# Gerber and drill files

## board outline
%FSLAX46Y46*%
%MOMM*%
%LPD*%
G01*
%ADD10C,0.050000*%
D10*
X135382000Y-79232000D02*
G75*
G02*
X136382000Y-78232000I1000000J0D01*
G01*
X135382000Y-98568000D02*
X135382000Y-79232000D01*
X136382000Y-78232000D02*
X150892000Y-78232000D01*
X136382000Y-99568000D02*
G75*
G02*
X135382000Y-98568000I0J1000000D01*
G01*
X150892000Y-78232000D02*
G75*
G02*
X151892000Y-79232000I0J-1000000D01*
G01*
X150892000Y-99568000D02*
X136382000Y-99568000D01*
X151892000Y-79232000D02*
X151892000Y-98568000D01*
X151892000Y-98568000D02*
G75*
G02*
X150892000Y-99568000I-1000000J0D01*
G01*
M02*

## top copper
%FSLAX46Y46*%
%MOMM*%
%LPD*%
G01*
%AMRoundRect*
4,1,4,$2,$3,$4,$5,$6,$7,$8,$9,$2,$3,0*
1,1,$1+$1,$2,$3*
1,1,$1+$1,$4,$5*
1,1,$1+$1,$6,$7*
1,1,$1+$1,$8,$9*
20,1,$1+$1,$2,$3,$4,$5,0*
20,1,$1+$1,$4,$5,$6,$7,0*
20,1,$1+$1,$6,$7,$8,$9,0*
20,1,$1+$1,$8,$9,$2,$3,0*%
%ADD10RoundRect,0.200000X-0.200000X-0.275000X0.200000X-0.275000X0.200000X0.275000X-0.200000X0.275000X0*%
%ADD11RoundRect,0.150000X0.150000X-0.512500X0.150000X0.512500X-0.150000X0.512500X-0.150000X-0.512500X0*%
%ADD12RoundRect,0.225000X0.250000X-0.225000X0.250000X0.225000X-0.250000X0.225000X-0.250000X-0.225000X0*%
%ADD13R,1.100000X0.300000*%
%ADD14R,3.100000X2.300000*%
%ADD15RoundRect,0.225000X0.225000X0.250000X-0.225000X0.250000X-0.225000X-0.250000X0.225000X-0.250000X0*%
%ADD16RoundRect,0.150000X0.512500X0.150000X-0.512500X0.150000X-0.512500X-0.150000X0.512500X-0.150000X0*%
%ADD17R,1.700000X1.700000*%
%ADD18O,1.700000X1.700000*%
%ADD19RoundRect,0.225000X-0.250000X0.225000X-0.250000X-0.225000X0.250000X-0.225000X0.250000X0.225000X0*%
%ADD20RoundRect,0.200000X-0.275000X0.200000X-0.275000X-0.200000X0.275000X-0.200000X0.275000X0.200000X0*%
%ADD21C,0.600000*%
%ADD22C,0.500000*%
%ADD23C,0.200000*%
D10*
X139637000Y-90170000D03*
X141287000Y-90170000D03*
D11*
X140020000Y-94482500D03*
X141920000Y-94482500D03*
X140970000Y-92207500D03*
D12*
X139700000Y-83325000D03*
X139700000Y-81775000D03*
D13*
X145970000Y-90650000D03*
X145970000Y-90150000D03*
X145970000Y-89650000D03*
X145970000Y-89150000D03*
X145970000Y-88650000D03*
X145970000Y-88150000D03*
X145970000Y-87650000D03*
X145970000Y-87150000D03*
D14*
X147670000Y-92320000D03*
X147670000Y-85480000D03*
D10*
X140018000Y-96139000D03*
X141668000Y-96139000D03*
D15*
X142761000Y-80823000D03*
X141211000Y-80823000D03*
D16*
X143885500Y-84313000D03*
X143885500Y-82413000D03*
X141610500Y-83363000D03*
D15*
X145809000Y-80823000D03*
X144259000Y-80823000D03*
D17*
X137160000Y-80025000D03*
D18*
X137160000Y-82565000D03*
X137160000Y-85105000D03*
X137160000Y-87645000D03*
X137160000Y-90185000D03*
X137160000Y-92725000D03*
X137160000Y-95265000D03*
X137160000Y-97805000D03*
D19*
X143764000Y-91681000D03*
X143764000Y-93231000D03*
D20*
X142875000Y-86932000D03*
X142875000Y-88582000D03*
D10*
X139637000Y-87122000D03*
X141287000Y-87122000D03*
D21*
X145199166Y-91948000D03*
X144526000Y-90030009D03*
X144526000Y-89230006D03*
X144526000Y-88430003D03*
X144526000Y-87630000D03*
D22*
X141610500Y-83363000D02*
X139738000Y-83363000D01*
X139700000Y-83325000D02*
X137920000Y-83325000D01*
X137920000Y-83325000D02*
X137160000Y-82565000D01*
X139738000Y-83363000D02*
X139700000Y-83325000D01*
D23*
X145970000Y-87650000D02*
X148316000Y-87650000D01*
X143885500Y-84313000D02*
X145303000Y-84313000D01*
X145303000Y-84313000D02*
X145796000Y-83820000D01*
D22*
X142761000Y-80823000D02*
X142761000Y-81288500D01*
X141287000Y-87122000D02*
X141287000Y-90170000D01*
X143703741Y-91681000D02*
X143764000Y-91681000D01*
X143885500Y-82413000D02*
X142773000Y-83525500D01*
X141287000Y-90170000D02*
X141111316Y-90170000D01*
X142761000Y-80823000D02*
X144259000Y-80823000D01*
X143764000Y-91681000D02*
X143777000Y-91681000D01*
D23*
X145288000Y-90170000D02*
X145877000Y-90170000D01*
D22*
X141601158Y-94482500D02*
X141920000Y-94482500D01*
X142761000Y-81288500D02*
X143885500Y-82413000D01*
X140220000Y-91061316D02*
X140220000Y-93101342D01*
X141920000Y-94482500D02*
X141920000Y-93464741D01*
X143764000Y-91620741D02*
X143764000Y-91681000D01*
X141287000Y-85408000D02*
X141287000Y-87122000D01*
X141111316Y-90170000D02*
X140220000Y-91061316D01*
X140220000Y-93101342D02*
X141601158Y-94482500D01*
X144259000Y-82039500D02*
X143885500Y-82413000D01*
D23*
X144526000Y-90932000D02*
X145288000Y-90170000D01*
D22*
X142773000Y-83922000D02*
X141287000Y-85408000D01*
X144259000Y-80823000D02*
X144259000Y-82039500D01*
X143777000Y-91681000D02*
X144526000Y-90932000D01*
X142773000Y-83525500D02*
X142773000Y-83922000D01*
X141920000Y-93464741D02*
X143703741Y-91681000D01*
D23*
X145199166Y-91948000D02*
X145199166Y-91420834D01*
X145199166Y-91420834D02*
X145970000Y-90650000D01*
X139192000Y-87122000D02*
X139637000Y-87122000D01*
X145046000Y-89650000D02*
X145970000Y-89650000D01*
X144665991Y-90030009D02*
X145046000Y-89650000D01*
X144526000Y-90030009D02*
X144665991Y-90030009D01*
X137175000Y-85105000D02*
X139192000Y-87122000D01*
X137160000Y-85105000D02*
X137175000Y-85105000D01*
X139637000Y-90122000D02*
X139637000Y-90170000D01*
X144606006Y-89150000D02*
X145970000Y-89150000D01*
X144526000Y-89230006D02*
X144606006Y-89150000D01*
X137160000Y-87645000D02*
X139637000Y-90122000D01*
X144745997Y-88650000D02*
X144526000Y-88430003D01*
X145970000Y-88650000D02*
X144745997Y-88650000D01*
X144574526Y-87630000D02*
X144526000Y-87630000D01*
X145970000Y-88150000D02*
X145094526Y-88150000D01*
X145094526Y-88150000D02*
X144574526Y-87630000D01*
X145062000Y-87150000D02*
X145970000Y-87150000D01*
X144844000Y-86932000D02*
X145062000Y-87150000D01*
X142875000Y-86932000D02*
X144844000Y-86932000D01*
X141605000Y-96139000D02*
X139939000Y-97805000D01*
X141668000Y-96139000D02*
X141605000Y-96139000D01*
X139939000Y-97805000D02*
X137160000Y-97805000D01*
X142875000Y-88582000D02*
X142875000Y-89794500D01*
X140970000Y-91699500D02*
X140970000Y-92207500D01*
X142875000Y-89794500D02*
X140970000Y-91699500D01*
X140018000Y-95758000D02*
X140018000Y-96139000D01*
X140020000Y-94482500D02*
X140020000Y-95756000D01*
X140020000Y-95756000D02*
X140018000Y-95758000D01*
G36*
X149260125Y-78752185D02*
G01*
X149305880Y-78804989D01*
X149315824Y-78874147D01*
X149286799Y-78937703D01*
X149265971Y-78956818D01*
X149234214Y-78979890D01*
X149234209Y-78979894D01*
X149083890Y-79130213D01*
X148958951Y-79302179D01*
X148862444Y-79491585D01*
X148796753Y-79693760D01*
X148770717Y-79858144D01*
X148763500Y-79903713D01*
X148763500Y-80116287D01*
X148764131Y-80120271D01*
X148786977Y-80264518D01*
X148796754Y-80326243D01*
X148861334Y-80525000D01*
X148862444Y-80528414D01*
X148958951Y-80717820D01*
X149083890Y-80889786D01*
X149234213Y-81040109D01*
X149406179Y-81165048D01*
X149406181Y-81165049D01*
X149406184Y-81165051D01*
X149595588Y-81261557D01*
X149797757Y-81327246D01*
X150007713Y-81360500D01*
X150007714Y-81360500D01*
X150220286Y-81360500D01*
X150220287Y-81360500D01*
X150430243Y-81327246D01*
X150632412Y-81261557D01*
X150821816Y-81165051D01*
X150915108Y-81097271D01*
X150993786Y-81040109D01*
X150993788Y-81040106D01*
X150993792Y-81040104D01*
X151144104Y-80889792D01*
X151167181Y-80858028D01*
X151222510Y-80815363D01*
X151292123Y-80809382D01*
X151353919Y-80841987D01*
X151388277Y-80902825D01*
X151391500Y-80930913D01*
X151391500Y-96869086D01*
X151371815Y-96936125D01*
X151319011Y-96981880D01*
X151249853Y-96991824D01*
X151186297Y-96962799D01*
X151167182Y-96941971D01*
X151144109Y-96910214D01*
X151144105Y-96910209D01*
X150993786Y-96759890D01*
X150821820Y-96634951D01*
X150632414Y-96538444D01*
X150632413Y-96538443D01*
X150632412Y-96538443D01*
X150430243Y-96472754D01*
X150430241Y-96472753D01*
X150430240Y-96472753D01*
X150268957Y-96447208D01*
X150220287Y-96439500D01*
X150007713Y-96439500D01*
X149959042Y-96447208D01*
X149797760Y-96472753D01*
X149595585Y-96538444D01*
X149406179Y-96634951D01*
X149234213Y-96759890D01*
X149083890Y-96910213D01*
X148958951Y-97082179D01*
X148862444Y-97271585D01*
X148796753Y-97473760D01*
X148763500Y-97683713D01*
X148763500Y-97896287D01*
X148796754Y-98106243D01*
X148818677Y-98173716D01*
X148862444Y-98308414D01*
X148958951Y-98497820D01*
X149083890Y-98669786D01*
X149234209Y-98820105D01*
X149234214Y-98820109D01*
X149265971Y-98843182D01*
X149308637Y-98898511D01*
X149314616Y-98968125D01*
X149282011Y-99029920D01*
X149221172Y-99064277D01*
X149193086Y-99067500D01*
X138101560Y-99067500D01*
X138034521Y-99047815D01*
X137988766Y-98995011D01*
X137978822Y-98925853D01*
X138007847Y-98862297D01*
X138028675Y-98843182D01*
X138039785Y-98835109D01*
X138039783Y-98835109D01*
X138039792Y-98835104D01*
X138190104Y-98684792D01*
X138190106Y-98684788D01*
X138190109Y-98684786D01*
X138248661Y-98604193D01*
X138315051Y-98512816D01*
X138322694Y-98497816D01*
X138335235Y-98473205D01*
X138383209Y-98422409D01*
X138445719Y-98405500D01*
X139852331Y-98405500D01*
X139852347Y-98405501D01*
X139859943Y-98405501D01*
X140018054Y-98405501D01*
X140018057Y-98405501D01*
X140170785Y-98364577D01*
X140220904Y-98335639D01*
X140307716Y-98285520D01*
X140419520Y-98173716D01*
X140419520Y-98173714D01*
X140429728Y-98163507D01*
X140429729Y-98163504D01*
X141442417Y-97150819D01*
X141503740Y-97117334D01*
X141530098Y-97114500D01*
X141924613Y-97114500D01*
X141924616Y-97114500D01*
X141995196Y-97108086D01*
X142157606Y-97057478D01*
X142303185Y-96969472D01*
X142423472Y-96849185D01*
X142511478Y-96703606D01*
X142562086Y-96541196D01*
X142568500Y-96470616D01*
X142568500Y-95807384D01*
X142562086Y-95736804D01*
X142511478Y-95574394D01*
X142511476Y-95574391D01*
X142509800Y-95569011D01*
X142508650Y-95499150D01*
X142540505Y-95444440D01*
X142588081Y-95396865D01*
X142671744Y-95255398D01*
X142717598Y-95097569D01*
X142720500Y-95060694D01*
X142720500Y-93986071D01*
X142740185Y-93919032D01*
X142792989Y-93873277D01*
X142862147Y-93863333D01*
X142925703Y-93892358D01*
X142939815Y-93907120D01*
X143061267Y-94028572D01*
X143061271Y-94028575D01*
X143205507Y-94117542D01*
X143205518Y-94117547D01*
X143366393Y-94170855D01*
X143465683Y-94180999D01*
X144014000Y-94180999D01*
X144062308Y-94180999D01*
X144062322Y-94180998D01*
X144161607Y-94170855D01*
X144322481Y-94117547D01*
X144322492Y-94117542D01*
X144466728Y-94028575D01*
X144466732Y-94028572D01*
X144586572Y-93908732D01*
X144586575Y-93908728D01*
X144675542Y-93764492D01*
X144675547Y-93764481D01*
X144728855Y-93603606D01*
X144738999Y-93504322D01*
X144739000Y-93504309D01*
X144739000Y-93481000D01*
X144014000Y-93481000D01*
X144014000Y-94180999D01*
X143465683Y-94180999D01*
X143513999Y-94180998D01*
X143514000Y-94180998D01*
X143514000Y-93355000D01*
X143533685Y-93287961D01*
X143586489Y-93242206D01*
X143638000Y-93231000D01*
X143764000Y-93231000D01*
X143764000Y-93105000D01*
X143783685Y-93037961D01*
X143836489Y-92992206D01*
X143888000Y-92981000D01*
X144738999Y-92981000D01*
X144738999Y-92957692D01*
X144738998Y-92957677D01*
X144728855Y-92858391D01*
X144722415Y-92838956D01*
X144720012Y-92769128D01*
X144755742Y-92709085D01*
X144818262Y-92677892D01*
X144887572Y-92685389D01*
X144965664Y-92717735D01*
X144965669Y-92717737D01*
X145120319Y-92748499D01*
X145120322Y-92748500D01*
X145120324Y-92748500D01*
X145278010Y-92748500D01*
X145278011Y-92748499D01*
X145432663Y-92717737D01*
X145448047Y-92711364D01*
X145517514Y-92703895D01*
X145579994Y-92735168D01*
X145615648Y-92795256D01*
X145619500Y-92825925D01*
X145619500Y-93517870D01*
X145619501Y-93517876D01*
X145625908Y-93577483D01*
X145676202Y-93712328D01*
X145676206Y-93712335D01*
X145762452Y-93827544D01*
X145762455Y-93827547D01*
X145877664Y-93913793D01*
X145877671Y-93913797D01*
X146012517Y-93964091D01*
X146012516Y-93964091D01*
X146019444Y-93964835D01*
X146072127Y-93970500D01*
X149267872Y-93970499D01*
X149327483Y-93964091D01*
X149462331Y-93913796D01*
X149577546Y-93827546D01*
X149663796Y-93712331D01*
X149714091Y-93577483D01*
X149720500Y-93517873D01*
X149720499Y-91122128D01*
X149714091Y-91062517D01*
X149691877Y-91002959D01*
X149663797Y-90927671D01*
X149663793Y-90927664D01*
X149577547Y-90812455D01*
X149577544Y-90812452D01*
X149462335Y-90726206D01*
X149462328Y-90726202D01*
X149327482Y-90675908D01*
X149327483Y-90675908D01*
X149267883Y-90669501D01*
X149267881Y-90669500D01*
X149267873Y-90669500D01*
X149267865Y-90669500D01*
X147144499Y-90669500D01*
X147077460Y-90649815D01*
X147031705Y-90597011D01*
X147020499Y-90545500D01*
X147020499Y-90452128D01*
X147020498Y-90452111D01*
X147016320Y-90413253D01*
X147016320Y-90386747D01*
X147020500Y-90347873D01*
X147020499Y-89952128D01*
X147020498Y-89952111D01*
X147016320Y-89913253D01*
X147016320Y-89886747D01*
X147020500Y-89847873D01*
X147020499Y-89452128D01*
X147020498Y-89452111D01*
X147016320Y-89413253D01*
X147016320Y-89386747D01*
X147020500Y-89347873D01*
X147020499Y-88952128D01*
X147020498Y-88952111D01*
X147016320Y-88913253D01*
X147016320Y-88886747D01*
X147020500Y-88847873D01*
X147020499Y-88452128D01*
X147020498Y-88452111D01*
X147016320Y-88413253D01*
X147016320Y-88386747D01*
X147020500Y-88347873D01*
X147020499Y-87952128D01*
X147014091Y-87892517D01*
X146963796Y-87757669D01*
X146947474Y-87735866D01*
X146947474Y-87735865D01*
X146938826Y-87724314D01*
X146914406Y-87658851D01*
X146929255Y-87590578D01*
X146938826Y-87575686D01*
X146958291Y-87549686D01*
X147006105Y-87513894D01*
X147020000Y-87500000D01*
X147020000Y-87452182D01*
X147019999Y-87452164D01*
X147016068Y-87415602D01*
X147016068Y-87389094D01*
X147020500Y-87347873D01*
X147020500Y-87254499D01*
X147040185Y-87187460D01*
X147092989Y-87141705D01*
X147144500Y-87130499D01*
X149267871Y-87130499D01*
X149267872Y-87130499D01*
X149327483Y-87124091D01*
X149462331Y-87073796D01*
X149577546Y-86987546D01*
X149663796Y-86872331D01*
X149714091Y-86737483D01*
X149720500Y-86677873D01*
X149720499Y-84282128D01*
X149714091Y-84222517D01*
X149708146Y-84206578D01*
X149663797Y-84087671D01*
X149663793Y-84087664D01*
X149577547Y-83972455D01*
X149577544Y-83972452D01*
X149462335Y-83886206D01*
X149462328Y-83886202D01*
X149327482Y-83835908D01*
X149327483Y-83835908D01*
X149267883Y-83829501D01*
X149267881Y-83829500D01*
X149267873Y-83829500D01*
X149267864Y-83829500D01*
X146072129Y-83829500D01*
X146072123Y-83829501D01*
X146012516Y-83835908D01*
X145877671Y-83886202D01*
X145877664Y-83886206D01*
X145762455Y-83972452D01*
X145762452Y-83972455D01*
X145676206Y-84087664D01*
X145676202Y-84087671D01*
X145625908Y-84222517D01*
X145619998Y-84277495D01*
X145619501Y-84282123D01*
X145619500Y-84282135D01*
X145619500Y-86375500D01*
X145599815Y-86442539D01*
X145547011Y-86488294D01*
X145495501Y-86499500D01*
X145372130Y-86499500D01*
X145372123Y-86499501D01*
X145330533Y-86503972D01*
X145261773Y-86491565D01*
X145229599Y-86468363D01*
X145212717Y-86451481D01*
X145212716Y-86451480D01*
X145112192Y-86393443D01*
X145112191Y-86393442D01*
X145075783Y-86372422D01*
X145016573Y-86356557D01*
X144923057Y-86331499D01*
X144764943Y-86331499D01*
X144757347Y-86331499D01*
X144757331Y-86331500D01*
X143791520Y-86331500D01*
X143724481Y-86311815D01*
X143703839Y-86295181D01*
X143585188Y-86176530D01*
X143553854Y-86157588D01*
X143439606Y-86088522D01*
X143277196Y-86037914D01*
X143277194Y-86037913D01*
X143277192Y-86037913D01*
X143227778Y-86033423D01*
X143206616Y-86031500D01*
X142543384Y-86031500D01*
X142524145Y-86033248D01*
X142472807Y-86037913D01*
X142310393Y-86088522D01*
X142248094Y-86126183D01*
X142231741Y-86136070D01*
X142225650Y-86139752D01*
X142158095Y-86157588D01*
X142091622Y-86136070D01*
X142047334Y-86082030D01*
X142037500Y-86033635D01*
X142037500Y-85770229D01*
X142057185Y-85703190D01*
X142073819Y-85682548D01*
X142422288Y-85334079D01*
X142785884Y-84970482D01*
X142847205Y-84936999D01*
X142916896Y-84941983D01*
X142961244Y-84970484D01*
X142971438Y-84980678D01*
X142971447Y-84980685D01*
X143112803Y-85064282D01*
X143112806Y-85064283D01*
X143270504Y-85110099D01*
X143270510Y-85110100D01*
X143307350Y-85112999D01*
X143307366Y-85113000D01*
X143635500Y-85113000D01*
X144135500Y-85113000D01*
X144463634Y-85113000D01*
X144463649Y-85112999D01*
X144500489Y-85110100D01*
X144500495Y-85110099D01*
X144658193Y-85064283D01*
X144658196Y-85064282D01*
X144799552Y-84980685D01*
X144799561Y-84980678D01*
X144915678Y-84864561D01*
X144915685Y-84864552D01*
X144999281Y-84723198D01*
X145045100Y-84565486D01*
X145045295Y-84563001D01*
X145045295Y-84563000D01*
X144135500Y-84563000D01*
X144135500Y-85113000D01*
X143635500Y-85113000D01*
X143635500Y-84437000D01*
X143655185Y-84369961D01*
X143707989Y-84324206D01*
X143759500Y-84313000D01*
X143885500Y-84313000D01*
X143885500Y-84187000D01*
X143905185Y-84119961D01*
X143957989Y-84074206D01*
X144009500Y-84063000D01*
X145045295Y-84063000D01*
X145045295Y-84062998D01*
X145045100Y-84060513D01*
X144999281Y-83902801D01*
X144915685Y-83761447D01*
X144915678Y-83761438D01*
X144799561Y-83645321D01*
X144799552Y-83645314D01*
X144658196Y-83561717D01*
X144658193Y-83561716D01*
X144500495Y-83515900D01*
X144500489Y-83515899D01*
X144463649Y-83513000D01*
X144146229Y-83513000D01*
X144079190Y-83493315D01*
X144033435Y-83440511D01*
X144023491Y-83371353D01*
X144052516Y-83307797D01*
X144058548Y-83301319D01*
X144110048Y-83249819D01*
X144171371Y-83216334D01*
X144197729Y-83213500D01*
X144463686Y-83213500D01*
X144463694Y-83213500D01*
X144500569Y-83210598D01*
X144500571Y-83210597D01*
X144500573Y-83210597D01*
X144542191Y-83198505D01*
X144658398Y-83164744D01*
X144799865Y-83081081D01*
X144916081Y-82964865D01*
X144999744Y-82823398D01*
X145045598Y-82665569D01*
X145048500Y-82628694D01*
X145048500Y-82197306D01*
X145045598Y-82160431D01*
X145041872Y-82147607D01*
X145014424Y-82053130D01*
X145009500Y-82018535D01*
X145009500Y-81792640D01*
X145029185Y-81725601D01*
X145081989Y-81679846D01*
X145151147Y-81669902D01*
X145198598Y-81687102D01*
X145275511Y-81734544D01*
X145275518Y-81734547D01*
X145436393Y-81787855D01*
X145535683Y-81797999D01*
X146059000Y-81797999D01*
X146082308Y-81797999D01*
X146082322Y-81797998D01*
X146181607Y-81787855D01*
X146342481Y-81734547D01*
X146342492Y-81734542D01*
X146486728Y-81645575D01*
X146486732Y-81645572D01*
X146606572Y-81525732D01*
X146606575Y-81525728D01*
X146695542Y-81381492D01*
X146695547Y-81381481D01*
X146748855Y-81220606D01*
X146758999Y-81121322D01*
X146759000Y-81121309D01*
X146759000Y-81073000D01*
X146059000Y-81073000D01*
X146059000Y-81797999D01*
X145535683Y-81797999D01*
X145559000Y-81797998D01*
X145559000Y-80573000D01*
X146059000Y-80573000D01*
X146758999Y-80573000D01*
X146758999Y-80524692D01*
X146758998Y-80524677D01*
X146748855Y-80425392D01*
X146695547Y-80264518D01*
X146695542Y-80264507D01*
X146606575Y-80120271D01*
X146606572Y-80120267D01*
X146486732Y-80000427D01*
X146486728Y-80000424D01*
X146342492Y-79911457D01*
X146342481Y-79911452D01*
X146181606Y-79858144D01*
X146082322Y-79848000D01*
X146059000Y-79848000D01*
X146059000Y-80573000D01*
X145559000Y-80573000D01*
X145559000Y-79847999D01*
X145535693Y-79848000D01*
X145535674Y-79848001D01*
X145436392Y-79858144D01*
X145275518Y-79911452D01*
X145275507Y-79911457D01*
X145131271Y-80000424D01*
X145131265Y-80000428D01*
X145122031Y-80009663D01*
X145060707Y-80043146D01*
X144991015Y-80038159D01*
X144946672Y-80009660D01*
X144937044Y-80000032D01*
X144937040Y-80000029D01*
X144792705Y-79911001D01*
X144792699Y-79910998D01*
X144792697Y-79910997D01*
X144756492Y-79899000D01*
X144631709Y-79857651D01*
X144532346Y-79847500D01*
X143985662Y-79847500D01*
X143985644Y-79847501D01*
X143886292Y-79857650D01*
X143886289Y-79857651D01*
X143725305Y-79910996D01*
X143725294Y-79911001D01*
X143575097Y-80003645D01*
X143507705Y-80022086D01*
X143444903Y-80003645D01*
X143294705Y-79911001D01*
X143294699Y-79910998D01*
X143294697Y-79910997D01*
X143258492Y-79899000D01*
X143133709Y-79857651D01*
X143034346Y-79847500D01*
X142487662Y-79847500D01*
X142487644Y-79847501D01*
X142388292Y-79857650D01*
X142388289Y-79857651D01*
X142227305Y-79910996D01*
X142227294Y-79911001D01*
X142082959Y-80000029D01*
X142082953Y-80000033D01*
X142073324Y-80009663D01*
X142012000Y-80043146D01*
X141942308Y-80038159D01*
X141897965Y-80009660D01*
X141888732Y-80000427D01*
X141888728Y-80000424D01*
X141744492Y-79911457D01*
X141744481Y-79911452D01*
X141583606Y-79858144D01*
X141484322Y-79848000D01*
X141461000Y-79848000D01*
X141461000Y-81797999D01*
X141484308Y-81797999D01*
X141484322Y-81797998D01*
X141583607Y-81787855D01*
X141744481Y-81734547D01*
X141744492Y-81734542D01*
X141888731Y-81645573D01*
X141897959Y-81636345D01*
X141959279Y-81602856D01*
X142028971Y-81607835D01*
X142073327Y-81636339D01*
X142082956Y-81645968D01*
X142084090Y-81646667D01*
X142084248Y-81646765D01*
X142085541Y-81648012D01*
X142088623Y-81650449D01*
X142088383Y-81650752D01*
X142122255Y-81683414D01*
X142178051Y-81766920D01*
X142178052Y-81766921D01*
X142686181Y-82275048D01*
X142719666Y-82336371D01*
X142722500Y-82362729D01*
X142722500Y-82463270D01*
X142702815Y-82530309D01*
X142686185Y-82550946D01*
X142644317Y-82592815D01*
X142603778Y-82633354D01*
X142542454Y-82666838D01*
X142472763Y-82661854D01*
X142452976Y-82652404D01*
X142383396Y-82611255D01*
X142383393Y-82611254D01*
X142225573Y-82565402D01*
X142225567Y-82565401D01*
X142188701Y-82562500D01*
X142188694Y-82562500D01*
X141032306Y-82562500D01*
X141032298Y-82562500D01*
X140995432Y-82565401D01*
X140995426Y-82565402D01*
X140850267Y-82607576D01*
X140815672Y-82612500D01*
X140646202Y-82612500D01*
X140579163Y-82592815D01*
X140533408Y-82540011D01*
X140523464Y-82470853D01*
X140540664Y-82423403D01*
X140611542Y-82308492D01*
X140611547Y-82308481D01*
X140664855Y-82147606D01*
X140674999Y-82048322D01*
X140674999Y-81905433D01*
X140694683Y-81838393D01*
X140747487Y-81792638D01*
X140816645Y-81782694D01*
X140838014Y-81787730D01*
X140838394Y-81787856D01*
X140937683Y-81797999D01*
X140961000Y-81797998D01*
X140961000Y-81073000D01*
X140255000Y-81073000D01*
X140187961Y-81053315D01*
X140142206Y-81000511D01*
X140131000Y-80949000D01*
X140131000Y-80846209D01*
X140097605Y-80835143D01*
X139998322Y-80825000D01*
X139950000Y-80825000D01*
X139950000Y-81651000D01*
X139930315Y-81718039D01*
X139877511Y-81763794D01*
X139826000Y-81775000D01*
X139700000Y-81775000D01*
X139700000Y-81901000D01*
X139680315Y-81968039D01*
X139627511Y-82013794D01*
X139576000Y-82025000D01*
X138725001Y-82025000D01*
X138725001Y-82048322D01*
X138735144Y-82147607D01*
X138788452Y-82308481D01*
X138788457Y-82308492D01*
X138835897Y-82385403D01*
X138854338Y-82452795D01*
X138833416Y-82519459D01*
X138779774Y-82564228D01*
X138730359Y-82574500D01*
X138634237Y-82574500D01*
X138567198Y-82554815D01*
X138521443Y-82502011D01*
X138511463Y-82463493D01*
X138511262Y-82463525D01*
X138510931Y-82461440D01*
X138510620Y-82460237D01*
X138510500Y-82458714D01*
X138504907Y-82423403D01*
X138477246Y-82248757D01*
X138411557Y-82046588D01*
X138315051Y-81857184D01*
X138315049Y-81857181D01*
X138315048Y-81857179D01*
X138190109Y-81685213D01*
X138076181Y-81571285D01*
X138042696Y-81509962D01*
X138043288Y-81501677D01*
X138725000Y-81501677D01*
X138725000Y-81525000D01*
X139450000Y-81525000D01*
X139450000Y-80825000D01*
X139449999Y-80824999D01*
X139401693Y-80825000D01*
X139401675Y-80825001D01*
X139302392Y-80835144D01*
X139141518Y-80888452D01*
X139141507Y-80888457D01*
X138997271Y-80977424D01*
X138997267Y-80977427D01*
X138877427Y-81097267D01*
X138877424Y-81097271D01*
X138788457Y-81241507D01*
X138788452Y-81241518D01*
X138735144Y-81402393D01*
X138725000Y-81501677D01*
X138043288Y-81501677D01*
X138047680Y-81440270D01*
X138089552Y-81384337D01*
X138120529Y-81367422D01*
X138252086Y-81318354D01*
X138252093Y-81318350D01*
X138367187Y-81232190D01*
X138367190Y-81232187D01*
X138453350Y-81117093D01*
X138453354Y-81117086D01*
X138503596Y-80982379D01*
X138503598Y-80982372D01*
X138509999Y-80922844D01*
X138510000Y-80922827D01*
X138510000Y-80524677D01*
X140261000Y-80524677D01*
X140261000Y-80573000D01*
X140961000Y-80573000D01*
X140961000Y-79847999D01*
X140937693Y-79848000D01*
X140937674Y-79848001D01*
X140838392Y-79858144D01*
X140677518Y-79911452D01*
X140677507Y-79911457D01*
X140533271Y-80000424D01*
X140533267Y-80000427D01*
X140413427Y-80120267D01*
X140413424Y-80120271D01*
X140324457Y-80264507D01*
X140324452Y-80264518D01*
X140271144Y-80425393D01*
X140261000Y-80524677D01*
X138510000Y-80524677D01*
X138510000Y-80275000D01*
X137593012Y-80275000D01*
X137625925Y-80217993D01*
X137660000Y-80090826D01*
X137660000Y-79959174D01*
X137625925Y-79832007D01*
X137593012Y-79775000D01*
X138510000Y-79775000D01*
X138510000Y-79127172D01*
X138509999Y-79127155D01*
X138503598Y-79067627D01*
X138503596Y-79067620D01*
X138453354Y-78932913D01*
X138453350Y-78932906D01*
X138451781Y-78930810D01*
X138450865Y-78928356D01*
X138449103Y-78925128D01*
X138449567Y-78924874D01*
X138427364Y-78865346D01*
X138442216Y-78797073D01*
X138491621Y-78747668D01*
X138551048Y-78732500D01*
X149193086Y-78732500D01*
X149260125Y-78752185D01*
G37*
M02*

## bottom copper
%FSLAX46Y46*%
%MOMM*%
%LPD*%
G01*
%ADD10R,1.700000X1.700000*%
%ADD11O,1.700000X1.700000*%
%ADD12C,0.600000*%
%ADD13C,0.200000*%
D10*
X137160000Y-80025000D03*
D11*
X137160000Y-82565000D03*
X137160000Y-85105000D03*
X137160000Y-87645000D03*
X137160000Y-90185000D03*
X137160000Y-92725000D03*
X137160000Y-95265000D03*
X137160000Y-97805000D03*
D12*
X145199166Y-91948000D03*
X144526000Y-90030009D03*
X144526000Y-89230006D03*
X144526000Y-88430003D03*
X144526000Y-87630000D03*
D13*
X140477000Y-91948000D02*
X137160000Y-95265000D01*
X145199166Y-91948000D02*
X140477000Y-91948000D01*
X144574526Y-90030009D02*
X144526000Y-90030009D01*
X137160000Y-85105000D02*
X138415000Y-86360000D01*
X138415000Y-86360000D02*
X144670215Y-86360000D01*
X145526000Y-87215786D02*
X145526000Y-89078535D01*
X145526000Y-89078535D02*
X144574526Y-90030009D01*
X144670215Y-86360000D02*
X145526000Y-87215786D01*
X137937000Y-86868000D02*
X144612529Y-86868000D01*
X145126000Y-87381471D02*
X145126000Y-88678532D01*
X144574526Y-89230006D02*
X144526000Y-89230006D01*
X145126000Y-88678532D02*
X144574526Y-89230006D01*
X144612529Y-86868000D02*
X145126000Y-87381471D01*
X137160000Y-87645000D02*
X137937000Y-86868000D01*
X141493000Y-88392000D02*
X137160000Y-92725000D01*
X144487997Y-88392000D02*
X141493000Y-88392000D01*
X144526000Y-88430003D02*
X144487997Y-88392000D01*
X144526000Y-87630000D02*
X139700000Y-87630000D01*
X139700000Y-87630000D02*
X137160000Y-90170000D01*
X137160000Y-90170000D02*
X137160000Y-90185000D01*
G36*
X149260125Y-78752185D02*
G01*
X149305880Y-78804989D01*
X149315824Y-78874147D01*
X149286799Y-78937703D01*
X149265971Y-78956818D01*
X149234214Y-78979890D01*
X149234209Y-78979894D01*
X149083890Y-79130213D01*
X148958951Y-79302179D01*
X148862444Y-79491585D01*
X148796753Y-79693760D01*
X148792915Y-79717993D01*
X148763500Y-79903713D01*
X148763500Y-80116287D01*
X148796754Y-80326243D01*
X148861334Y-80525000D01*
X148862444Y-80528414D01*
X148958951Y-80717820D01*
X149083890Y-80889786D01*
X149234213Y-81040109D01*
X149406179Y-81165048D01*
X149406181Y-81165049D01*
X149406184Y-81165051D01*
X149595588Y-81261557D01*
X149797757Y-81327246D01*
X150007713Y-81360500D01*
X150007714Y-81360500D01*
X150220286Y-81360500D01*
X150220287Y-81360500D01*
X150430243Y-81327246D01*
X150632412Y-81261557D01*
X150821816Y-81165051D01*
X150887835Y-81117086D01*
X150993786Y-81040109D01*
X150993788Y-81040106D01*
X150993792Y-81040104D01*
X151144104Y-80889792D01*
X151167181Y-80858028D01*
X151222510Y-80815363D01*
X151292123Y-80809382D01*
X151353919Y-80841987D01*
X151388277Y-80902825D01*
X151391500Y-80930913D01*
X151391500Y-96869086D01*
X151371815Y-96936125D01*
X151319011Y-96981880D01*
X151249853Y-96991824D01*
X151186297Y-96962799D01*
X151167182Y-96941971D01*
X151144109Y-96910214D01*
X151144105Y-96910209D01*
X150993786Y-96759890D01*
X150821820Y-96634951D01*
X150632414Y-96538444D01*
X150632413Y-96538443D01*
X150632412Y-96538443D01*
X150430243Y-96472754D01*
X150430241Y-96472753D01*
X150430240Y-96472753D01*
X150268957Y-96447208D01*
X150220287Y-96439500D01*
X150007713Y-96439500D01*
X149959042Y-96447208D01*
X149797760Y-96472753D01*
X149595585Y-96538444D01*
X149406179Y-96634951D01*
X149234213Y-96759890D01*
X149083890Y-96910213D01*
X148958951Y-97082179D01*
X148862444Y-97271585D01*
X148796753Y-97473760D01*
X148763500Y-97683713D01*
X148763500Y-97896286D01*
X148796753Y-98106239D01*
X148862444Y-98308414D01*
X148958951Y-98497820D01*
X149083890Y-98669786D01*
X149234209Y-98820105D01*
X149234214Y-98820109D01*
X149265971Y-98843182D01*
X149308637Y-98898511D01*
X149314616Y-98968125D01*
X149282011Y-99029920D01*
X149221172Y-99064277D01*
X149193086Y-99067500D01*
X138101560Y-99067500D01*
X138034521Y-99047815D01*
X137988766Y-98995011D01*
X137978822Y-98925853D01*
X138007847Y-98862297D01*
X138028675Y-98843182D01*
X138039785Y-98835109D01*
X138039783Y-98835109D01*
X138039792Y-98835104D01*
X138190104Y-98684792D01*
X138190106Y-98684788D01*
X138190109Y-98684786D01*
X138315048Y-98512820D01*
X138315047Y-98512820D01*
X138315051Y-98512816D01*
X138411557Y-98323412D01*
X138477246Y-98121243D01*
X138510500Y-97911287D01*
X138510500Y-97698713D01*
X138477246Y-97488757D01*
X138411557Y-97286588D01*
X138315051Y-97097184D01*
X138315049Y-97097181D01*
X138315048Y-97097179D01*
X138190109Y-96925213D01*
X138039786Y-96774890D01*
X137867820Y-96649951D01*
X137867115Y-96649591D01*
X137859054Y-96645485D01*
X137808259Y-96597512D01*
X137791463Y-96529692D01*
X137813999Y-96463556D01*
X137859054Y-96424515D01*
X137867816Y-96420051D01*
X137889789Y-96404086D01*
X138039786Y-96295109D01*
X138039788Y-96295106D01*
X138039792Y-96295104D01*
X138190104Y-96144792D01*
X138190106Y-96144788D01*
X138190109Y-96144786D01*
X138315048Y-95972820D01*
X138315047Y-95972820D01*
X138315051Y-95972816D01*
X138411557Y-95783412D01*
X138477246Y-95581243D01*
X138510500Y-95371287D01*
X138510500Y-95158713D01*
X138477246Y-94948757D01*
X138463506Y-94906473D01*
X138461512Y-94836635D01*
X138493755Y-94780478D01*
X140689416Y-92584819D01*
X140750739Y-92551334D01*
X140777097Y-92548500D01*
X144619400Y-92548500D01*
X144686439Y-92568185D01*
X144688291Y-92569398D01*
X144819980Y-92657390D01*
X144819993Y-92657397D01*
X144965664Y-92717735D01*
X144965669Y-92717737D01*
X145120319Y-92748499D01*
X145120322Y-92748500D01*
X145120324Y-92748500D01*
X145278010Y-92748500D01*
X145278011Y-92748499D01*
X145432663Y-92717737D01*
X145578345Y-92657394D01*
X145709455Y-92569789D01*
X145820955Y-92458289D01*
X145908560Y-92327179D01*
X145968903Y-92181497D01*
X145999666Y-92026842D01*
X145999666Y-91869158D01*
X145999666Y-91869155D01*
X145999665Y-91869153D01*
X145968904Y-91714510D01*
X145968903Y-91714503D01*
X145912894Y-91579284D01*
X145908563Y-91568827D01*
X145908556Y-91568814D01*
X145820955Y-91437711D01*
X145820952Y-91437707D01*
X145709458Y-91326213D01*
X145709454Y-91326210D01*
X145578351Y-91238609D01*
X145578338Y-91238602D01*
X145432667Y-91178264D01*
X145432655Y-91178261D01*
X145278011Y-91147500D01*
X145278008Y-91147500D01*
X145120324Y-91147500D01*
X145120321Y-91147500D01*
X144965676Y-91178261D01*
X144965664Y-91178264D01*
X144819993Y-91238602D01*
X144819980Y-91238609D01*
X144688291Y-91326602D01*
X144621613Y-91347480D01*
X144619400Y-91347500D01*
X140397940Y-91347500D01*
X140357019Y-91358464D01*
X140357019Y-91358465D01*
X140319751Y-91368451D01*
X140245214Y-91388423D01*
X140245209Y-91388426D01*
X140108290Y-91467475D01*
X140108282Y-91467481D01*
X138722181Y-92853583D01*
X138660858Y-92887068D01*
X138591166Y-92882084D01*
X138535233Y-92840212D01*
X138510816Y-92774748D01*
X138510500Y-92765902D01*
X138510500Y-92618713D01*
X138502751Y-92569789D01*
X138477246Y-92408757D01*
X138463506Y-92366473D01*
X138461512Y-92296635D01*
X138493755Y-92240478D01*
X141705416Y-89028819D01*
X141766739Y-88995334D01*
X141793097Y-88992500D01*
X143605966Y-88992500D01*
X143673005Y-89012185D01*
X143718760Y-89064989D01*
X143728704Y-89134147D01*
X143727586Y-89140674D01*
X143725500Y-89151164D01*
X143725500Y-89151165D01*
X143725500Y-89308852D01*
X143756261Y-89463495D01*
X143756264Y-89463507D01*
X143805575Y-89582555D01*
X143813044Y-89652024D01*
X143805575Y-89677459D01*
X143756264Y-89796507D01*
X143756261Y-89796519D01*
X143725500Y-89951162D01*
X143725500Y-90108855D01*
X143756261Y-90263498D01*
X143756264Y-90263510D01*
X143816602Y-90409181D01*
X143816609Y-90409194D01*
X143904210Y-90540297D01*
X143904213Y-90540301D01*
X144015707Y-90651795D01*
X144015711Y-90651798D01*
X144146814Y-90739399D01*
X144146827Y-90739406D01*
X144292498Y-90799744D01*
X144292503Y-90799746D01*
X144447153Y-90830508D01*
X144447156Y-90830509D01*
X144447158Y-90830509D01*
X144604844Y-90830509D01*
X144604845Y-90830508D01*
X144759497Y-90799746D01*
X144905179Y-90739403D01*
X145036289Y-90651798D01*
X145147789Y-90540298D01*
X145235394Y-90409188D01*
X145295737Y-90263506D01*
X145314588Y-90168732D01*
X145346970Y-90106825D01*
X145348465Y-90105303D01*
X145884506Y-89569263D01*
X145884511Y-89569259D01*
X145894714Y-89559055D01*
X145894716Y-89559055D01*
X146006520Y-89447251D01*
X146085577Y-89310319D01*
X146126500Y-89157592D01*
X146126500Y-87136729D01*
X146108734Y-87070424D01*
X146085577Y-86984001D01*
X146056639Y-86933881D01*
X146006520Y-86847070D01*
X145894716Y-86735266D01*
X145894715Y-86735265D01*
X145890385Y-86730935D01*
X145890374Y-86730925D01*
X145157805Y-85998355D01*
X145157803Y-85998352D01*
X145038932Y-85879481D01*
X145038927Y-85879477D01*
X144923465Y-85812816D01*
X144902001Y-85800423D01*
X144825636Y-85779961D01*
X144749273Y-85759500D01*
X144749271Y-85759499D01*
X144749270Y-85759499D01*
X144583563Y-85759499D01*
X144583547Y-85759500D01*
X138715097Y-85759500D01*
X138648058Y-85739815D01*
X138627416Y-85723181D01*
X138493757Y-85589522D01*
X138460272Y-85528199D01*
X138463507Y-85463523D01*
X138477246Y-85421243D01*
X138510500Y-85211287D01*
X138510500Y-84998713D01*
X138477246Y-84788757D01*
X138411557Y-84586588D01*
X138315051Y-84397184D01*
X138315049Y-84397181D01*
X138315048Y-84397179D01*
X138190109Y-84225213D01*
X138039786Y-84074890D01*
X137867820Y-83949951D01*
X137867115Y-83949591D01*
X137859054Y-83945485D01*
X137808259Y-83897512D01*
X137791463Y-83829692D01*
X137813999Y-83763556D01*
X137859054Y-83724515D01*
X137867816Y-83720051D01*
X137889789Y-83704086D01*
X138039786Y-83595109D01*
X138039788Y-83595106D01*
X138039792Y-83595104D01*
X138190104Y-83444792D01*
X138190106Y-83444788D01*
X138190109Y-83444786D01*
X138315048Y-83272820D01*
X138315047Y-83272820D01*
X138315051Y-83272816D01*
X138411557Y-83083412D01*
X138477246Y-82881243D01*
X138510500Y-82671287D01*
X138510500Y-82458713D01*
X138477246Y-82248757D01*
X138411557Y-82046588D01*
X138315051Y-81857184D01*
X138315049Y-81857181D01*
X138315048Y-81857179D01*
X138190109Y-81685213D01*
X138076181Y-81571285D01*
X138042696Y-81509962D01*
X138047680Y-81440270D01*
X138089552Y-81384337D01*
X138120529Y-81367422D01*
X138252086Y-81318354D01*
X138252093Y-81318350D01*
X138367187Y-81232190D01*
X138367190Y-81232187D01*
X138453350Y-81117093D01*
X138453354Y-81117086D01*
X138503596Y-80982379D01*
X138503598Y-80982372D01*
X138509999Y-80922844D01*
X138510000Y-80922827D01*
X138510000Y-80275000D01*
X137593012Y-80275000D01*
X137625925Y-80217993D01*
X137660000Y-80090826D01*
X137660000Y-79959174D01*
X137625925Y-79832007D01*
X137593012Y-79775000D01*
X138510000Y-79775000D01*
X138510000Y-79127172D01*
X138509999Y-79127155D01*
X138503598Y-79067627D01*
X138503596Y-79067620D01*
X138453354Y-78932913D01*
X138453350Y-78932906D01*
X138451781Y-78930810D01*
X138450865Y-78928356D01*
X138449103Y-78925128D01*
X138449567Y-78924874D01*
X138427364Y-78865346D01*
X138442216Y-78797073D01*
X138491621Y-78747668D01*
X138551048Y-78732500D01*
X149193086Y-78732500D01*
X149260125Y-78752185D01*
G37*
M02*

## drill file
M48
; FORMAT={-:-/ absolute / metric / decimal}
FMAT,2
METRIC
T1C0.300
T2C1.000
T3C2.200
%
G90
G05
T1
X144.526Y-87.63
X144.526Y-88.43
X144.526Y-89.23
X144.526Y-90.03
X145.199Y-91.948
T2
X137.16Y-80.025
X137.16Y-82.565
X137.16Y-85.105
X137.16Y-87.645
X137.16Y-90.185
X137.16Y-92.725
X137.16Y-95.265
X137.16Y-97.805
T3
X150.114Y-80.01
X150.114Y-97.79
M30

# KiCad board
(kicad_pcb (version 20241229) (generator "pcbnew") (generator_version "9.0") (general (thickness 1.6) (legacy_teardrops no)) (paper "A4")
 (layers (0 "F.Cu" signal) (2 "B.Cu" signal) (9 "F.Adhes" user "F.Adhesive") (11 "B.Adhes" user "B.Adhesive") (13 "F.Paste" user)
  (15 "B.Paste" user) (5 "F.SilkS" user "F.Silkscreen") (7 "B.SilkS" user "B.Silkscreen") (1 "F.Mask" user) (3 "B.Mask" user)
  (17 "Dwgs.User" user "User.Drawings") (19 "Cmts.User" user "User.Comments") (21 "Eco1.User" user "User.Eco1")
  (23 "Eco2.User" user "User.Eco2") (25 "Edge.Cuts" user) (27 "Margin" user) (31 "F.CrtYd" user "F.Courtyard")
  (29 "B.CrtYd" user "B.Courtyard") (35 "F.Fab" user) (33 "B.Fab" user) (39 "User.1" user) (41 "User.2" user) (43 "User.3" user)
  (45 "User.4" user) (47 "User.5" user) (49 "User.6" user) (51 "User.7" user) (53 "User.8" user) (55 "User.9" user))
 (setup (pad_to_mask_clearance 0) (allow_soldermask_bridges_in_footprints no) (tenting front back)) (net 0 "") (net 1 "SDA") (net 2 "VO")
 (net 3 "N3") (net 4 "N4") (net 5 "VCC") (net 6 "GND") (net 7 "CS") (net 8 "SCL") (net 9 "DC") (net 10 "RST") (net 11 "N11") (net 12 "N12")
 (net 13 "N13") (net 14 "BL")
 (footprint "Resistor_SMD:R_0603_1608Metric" (layer "F.Cu") (at 140.462 90.17)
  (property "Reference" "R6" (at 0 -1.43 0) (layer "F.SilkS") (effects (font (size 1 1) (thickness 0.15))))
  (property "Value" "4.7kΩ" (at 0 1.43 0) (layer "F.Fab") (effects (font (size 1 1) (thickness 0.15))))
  (pad "1" smd roundrect (at -0.825 0) (size 0.8 0.95) (layers "F.Cu" "F.Mask" "F.Paste") (roundrect_rratio 0.25) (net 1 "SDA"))
  (pad "2" smd roundrect (at 0.825 0) (size 0.8 0.95) (layers "F.Cu" "F.Mask" "F.Paste") (roundrect_rratio 0.25) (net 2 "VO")))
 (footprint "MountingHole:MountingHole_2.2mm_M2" (layer "F.Cu") (at 150.114 97.79)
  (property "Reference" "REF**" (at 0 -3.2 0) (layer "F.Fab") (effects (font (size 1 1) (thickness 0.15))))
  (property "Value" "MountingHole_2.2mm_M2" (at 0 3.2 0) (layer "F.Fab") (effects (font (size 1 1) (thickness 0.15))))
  (pad "" np_thru_hole circle (at 0 0) (size 2.2 2.2) (drill 2.2) (layers "*.Cu" "*.Mask")))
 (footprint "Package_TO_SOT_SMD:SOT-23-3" (layer "F.Cu") (at 140.97 93.345 90)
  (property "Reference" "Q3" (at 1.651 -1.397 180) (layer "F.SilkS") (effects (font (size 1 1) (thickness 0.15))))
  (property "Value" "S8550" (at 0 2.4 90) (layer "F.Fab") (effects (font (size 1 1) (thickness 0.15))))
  (pad "1" smd roundrect (at -1.1375 -0.95 90) (size 1.325 0.6) (layers "F.Cu" "F.Mask" "F.Paste") (roundrect_rratio 0.25) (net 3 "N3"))
  (pad "2" smd roundrect (at -1.1375 0.95 90) (size 1.325 0.6) (layers "F.Cu" "F.Mask" "F.Paste") (roundrect_rratio 0.25) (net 2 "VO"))
  (pad "3" smd roundrect (at 1.1375 0 90) (size 1.325 0.6) (layers "F.Cu" "F.Mask" "F.Paste") (roundrect_rratio 0.25) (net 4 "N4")))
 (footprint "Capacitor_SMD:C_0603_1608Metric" (layer "F.Cu") (at 139.7 82.55 90)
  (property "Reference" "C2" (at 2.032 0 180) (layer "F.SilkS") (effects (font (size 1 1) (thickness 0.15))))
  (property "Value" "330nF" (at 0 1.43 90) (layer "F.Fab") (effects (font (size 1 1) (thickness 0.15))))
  (pad "1" smd roundrect (at -0.775 0 90) (size 0.9 0.95) (layers "F.Cu" "F.Mask" "F.Paste") (roundrect_rratio 0.25) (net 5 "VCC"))
  (pad "2" smd roundrect (at 0.775 0 90) (size 0.9 0.95) (layers "F.Cu" "F.Mask" "F.Paste") (roundrect_rratio 0.25) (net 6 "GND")))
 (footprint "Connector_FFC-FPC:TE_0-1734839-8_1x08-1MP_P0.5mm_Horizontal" (layer "F.Cu") (at 147.32 88.9 90)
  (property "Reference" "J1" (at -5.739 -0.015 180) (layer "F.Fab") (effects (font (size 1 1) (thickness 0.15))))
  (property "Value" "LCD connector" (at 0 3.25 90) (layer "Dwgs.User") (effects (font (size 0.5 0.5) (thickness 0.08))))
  (pad "1" smd rect (at -1.75 -1.35 90) (size 0.3 1.1) (layers "F.Cu" "F.Mask" "F.Paste") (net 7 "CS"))
  (pad "2" smd rect (at -1.25 -1.35 90) (size 0.3 1.1) (layers "F.Cu" "F.Mask" "F.Paste") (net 2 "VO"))
  (pad "3" smd rect (at -0.75 -1.35 90) (size 0.3 1.1) (layers "F.Cu" "F.Mask" "F.Paste") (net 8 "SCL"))
  (pad "4" smd rect (at -0.25 -1.35 90) (size 0.3 1.1) (layers "F.Cu" "F.Mask" "F.Paste") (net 1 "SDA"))
  (pad "5" smd rect (at 0.25 -1.35 90) (size 0.3 1.1) (layers "F.Cu" "F.Mask" "F.Paste") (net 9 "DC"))
  (pad "6" smd rect (at 0.75 -1.35 90) (size 0.3 1.1) (layers "F.Cu" "F.Mask" "F.Paste") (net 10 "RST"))
  (pad "7" smd rect (at 1.25 -1.35 90) (size 0.3 1.1) (layers "F.Cu" "F.Mask" "F.Paste") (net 6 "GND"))
  (pad "8" smd rect (at 1.75 -1.35 90) (size 0.3 1.1) (layers "F.Cu" "F.Mask" "F.Paste") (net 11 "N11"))
  (pad "MP" smd rect (at -3.42 0.35 90) (size 2.3 3.1) (layers "F.Cu" "F.Mask" "F.Paste") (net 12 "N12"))
  (pad "MP" smd rect (at 3.42 0.35 90) (size 2.3 3.1) (layers "F.Cu" "F.Mask" "F.Paste") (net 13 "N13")))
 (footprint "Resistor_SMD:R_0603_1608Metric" (layer "F.Cu") (at 140.843 96.139)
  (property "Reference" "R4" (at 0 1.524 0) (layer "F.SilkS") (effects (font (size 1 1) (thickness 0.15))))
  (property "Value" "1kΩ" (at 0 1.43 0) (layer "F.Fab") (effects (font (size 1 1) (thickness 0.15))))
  (pad "1" smd roundrect (at -0.825 0) (size 0.8 0.95) (layers "F.Cu" "F.Mask" "F.Paste") (roundrect_rratio 0.25) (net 3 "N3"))
  (pad "2" smd roundrect (at 0.825 0) (size 0.8 0.95) (layers "F.Cu" "F.Mask" "F.Paste") (roundrect_rratio 0.25) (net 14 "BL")))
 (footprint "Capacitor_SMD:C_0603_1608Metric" (layer "F.Cu") (at 141.986 80.823 180)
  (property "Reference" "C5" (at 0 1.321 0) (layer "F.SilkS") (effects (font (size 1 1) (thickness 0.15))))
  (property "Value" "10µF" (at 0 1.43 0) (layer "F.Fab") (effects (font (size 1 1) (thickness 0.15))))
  (pad "1" smd roundrect (at -0.775 0 180) (size 0.9 0.95) (layers "F.Cu" "F.Mask" "F.Paste") (roundrect_rratio 0.25) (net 2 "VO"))
  (pad "2" smd roundrect (at 0.775 0 180) (size 0.9 0.95) (layers "F.Cu" "F.Mask" "F.Paste") (roundrect_rratio 0.25) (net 6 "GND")))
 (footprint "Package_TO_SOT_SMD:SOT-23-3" (layer "F.Cu") (at 142.748 83.363 180)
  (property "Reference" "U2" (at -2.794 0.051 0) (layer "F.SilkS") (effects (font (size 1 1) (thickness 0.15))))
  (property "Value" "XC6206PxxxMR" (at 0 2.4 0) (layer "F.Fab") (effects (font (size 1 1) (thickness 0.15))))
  (pad "1" smd roundrect (at -1.1375 -0.95 180) (size 1.325 0.6) (layers "F.Cu" "F.Mask" "F.Paste") (roundrect_rratio 0.25) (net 6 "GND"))
  (pad "2" smd roundrect (at -1.1375 0.95 180) (size 1.325 0.6) (layers "F.Cu" "F.Mask" "F.Paste") (roundrect_rratio 0.25) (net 2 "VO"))
  (pad "3" smd roundrect (at 1.1375 0 180) (size 1.325 0.6) (layers "F.Cu" "F.Mask" "F.Paste") (roundrect_rratio 0.25) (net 5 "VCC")))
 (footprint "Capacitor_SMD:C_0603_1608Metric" (layer "F.Cu") (at 145.034 80.823 180)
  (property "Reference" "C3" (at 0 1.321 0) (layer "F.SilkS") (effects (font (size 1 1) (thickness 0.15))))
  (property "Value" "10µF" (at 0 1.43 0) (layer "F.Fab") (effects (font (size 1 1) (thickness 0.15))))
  (pad "1" smd roundrect (at -0.775 0 180) (size 0.9 0.95) (layers "F.Cu" "F.Mask" "F.Paste") (roundrect_rratio 0.25) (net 6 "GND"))
  (pad "2" smd roundrect (at 0.775 0 180) (size 0.9 0.95) (layers "F.Cu" "F.Mask" "F.Paste") (roundrect_rratio 0.25) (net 2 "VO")))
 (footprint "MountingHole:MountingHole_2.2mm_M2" (layer "F.Cu") (at 150.114 80.01)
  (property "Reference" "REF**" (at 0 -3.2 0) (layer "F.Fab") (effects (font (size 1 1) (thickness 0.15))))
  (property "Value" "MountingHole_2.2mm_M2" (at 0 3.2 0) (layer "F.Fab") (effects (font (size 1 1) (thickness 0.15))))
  (pad "" np_thru_hole circle (at 0 0) (size 2.2 2.2) (drill 2.2) (layers "*.Cu" "*.Mask")))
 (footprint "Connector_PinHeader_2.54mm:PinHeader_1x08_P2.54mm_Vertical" (layer "F.Cu") (at 137.16 80.025)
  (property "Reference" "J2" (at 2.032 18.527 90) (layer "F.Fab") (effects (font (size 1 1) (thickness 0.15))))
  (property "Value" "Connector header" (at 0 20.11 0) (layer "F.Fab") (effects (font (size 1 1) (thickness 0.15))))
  (pad "1" thru_hole rect (at 0 0) (size 1.7 1.7) (drill 1) (layers "*.Cu" "*.Mask") (remove_unused_layers no) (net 6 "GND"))
  (pad "2" thru_hole oval (at 0 2.54) (size 1.7 1.7) (drill 1) (layers "*.Cu" "*.Mask") (remove_unused_layers no) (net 5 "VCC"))
  (pad "3" thru_hole oval (at 0 5.08) (size 1.7 1.7) (drill 1) (layers "*.Cu" "*.Mask") (remove_unused_layers no) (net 8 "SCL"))
  (pad "4" thru_hole oval (at 0 7.62) (size 1.7 1.7) (drill 1) (layers "*.Cu" "*.Mask") (remove_unused_layers no) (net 1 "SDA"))
  (pad "5" thru_hole oval (at 0 10.16) (size 1.7 1.7) (drill 1) (layers "*.Cu" "*.Mask") (remove_unused_layers no) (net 10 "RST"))
  (pad "6" thru_hole oval (at 0 12.7) (size 1.7 1.7) (drill 1) (layers "*.Cu" "*.Mask") (remove_unused_layers no) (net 9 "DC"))
  (pad "7" thru_hole oval (at 0 15.24) (size 1.7 1.7) (drill 1) (layers "*.Cu" "*.Mask") (remove_unused_layers no) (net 7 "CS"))
  (pad "8" thru_hole oval (at 0 17.78) (size 1.7 1.7) (drill 1) (layers "*.Cu" "*.Mask") (remove_unused_layers no) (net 14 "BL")))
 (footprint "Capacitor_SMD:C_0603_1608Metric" (layer "F.Cu") (at 143.764 92.456 -90)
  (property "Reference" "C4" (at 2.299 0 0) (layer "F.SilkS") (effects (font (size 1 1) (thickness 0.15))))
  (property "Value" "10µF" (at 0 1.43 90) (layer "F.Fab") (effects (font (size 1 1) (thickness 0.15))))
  (pad "1" smd roundrect (at -0.775 0 270) (size 0.9 0.95) (layers "F.Cu" "F.Mask" "F.Paste") (roundrect_rratio 0.25) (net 2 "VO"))
  (pad "2" smd roundrect (at 0.775 0 270) (size 0.9 0.95) (layers "F.Cu" "F.Mask" "F.Paste") (roundrect_rratio 0.25) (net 6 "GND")))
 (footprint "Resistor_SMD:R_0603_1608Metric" (layer "F.Cu") (at 142.875 87.757 -90)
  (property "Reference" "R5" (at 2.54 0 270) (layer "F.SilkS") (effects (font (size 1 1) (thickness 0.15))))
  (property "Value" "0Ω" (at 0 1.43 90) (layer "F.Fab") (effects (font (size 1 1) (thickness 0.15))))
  (pad "1" smd roundrect (at -0.825 0 270) (size 0.8 0.95) (layers "F.Cu" "F.Mask" "F.Paste") (roundrect_rratio 0.25) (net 11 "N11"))
  (pad "2" smd roundrect (at 0.825 0 270) (size 0.8 0.95) (layers "F.Cu" "F.Mask" "F.Paste") (roundrect_rratio 0.25) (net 4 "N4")))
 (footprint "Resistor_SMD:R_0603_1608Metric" (layer "F.Cu") (at 140.462 87.122)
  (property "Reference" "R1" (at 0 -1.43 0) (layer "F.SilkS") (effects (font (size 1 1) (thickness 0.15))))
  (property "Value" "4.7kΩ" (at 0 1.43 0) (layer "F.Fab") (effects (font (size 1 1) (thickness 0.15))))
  (pad "1" smd roundrect (at -0.825 0) (size 0.8 0.95) (layers "F.Cu" "F.Mask" "F.Paste") (roundrect_rratio 0.25) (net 8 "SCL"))
  (pad "2" smd roundrect (at 0.825 0) (size 0.8 0.95) (layers "F.Cu" "F.Mask" "F.Paste") (roundrect_rratio 0.25) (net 2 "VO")))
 (gr_arc (start 135.382 79.232) (mid 135.674893 78.524893) (end 136.382 78.232) (stroke (width 0.05) (type default)) (layer "Edge.Cuts"))
 (gr_line (start 135.382 98.568) (end 135.382 79.232) (stroke (width 0.05) (type default)) (layer "Edge.Cuts"))
 (gr_line (start 136.382 78.232) (end 150.892 78.232) (stroke (width 0.05) (type default)) (layer "Edge.Cuts"))
 (gr_arc (start 136.382 99.568) (mid 135.674893 99.275107) (end 135.382 98.568) (stroke (width 0.05) (type default)) (layer "Edge.Cuts"))
 (gr_arc (start 150.892 78.232) (mid 151.599107 78.524893) (end 151.892 79.232) (stroke (width 0.05) (type default)) (layer "Edge.Cuts"))
 (gr_line (start 150.892 99.568) (end 136.382 99.568) (stroke (width 0.05) (type default)) (layer "Edge.Cuts"))
 (gr_line (start 151.892 79.232) (end 151.892 98.568) (stroke (width 0.05) (type default)) (layer "Edge.Cuts"))
 (gr_arc (start 151.892 98.568) (mid 151.599107 99.275107) (end 150.892 99.568) (stroke (width 0.05) (type default)) (layer "Edge.Cuts"))
 (segment (start 141.6105 83.363) (end 139.738 83.363) (width 0.5) (layer "F.Cu") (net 5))
 (segment (start 139.7 83.325) (end 137.92 83.325) (width 0.5) (layer "F.Cu") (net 5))
 (segment (start 137.92 83.325) (end 137.16 82.565) (width 0.5) (layer "F.Cu") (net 5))
 (segment (start 139.738 83.363) (end 139.7 83.325) (width 0.5) (layer "F.Cu") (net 5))
 (segment (start 145.97 87.65) (end 148.316 87.65) (width 0.2) (layer "F.Cu") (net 6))
 (segment (start 143.8855 84.313) (end 145.303 84.313) (width 0.2) (layer "F.Cu") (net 6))
 (segment (start 145.303 84.313) (end 145.796 83.82) (width 0.2) (layer "F.Cu") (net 6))
 (segment (start 142.761 80.823) (end 142.761 81.2885) (width 0.5) (layer "F.Cu") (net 2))
 (segment (start 141.287 87.122) (end 141.287 90.17) (width 0.5) (layer "F.Cu") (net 2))
 (segment (start 143.703741 91.681) (end 143.764 91.681) (width 0.5) (layer "F.Cu") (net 2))
 (segment (start 143.8855 82.413) (end 142.773 83.5255) (width 0.5) (layer "F.Cu") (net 2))
 (segment (start 141.287 90.17) (end 141.111316 90.17) (width 0.5) (layer "F.Cu") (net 2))
 (segment (start 142.761 80.823) (end 144.259 80.823) (width 0.5) (layer "F.Cu") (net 2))
 (segment (start 143.764 91.681) (end 143.777 91.681) (width 0.5) (layer "F.Cu") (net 2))
 (segment (start 145.288 90.17) (end 145.877 90.17) (width 0.2) (layer "F.Cu") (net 2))
 (segment (start 141.601158 94.4825) (end 141.92 94.4825) (width 0.5) (layer "F.Cu") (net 2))
 (segment (start 142.761 81.2885) (end 143.8855 82.413) (width 0.5) (layer "F.Cu") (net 2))
 (segment (start 140.22 91.061316) (end 140.22 93.101342) (width 0.5) (layer "F.Cu") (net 2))
 (segment (start 141.92 94.4825) (end 141.92 93.464741) (width 0.5) (layer "F.Cu") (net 2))
 (segment (start 143.764 91.620741) (end 143.764 91.681) (width 0.5) (layer "F.Cu") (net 2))
 (segment (start 141.287 85.408) (end 141.287 87.122) (width 0.5) (layer "F.Cu") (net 2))
 (segment (start 141.111316 90.17) (end 140.22 91.061316) (width 0.5) (layer "F.Cu") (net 2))
 (segment (start 140.22 93.101342) (end 141.601158 94.4825) (width 0.5) (layer "F.Cu") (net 2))
 (segment (start 144.259 82.0395) (end 143.8855 82.413) (width 0.5) (layer "F.Cu") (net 2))
 (segment (start 144.526 90.932) (end 145.288 90.17) (width 0.2) (layer "F.Cu") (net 2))
 (segment (start 142.773 83.922) (end 141.287 85.408) (width 0.5) (layer "F.Cu") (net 2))
 (segment (start 144.259 80.823) (end 144.259 82.0395) (width 0.5) (layer "F.Cu") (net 2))
 (segment (start 143.777 91.681) (end 144.526 90.932) (width 0.5) (layer "F.Cu") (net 2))
 (segment (start 142.773 83.5255) (end 142.773 83.922) (width 0.5) (layer "F.Cu") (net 2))
 (segment (start 141.92 93.464741) (end 143.703741 91.681) (width 0.5) (layer "F.Cu") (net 2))
 (segment (start 145.199166 91.948) (end 145.199166 91.420834) (width 0.2) (layer "F.Cu") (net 7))
 (segment (start 145.199166 91.420834) (end 145.97 90.65) (width 0.2) (layer "F.Cu") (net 7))
 (via (at 145.199166 91.948) (size 0.6) (drill 0.3) (layers "F.Cu" "B.Cu") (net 7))
 (segment (start 140.477 91.948) (end 137.16 95.265) (width 0.2) (layer "B.Cu") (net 7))
 (segment (start 145.199166 91.948) (end 140.477 91.948) (width 0.2) (layer "B.Cu") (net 7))
 (segment (start 139.192 87.122) (end 139.637 87.122) (width 0.2) (layer "F.Cu") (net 8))
 (segment (start 145.046 89.65) (end 145.97 89.65) (width 0.2) (layer "F.Cu") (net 8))
 (segment (start 144.665991 90.030009) (end 145.046 89.65) (width 0.2) (layer "F.Cu") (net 8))
 (segment (start 144.526 90.030009) (end 144.665991 90.030009) (width 0.2) (layer "F.Cu") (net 8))
 (segment (start 137.175 85.105) (end 139.192 87.122) (width 0.2) (layer "F.Cu") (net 8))
 (segment (start 137.16 85.105) (end 137.175 85.105) (width 0.2) (layer "F.Cu") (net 8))
 (via (at 144.526 90.030009) (size 0.6) (drill 0.3) (layers "F.Cu" "B.Cu") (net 8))
 (segment (start 144.574526 90.030009) (end 144.526 90.030009) (width 0.2) (layer "B.Cu") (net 8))
 (segment (start 137.16 85.105) (end 138.415 86.36) (width 0.2) (layer "B.Cu") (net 8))
 (segment (start 138.415 86.36) (end 144.670215 86.36) (width 0.2) (layer "B.Cu") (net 8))
 (segment (start 145.526 87.215786) (end 145.526 89.078535) (width 0.2) (layer "B.Cu") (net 8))
 (segment (start 145.526 89.078535) (end 144.574526 90.030009) (width 0.2) (layer "B.Cu") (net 8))
 (segment (start 144.670215 86.36) (end 145.526 87.215786) (width 0.2) (layer "B.Cu") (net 8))
 (segment (start 139.637 90.122) (end 139.637 90.17) (width 0.2) (layer "F.Cu") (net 1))
 (segment (start 144.606006 89.15) (end 145.97 89.15) (width 0.2) (layer "F.Cu") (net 1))
 (segment (start 144.526 89.230006) (end 144.606006 89.15) (width 0.2) (layer "F.Cu") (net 1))
 (segment (start 137.16 87.645) (end 139.637 90.122) (width 0.2) (layer "F.Cu") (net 1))
 (via (at 144.526 89.230006) (size 0.6) (drill 0.3) (layers "F.Cu" "B.Cu") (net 1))
 (segment (start 137.937 86.868) (end 144.612529 86.868) (width 0.2) (layer "B.Cu") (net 1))
 (segment (start 145.126 87.381471) (end 145.126 88.678532) (width 0.2) (layer "B.Cu") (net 1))
 (segment (start 144.574526 89.230006) (end 144.526 89.230006) (width 0.2) (layer "B.Cu") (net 1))
 (segment (start 145.126 88.678532) (end 144.574526 89.230006) (width 0.2) (layer "B.Cu") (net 1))
 (segment (start 144.612529 86.868) (end 145.126 87.381471) (width 0.2) (layer "B.Cu") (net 1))
 (segment (start 137.16 87.645) (end 137.937 86.868) (width 0.2) (layer "B.Cu") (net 1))
 (segment (start 144.745997 88.65) (end 144.526 88.430003) (width 0.2) (layer "F.Cu") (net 9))
 (segment (start 145.97 88.65) (end 144.745997 88.65) (width 0.2) (layer "F.Cu") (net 9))
 (via (at 144.526 88.430003) (size 0.6) (drill 0.3) (layers "F.Cu" "B.Cu") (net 9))
 (segment (start 141.493 88.392) (end 137.16 92.725) (width 0.2) (layer "B.Cu") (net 9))
 (segment (start 144.487997 88.392) (end 141.493 88.392) (width 0.2) (layer "B.Cu") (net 9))
 (segment (start 144.526 88.430003) (end 144.487997 88.392) (width 0.2) (layer "B.Cu") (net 9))
 (segment (start 144.574526 87.63) (end 144.526 87.63) (width 0.2) (layer "F.Cu") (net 10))
 (segment (start 145.97 88.15) (end 145.094526 88.15) (width 0.2) (layer "F.Cu") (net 10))
 (segment (start 145.094526 88.15) (end 144.574526 87.63) (width 0.2) (layer "F.Cu") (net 10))
 (via (at 144.526 87.63) (size 0.6) (drill 0.3) (layers "F.Cu" "B.Cu") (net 10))
 (segment (start 144.526 87.63) (end 139.7 87.63) (width 0.2) (layer "B.Cu") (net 10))
 (segment (start 139.7 87.63) (end 137.16 90.17) (width 0.2) (layer "B.Cu") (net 10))
 (segment (start 137.16 90.17) (end 137.16 90.185) (width 0.2) (layer "B.Cu") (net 10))
 (segment (start 145.062 87.15) (end 145.97 87.15) (width 0.2) (layer "F.Cu") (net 11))
 (segment (start 144.844 86.932) (end 145.062 87.15) (width 0.2) (layer "F.Cu") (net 11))
 (segment (start 142.875 86.932) (end 144.844 86.932) (width 0.2) (layer "F.Cu") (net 11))
 (segment (start 141.605 96.139) (end 139.939 97.805) (width 0.2) (layer "F.Cu") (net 14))
 (segment (start 141.668 96.139) (end 141.605 96.139) (width 0.2) (layer "F.Cu") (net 14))
 (segment (start 139.939 97.805) (end 137.16 97.805) (width 0.2) (layer "F.Cu") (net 14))
 (segment (start 142.875 88.582) (end 142.875 89.7945) (width 0.2) (layer "F.Cu") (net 4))
 (segment (start 140.97 91.6995) (end 140.97 92.2075) (width 0.2) (layer "F.Cu") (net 4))
 (segment (start 142.875 89.7945) (end 140.97 91.6995) (width 0.2) (layer "F.Cu") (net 4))
 (segment (start 140.018 95.758) (end 140.018 96.139) (width 0.2) (layer "F.Cu") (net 3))
 (segment (start 140.02 94.4825) (end 140.02 95.756) (width 0.2) (layer "F.Cu") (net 3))
 (segment (start 140.02 95.756) (end 140.018 95.758) (width 0.2) (layer "F.Cu") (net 3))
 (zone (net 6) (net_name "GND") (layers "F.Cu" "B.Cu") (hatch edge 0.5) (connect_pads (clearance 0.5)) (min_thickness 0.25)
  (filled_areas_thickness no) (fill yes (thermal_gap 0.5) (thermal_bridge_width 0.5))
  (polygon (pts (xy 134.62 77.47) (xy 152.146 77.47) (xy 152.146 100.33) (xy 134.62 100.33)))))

